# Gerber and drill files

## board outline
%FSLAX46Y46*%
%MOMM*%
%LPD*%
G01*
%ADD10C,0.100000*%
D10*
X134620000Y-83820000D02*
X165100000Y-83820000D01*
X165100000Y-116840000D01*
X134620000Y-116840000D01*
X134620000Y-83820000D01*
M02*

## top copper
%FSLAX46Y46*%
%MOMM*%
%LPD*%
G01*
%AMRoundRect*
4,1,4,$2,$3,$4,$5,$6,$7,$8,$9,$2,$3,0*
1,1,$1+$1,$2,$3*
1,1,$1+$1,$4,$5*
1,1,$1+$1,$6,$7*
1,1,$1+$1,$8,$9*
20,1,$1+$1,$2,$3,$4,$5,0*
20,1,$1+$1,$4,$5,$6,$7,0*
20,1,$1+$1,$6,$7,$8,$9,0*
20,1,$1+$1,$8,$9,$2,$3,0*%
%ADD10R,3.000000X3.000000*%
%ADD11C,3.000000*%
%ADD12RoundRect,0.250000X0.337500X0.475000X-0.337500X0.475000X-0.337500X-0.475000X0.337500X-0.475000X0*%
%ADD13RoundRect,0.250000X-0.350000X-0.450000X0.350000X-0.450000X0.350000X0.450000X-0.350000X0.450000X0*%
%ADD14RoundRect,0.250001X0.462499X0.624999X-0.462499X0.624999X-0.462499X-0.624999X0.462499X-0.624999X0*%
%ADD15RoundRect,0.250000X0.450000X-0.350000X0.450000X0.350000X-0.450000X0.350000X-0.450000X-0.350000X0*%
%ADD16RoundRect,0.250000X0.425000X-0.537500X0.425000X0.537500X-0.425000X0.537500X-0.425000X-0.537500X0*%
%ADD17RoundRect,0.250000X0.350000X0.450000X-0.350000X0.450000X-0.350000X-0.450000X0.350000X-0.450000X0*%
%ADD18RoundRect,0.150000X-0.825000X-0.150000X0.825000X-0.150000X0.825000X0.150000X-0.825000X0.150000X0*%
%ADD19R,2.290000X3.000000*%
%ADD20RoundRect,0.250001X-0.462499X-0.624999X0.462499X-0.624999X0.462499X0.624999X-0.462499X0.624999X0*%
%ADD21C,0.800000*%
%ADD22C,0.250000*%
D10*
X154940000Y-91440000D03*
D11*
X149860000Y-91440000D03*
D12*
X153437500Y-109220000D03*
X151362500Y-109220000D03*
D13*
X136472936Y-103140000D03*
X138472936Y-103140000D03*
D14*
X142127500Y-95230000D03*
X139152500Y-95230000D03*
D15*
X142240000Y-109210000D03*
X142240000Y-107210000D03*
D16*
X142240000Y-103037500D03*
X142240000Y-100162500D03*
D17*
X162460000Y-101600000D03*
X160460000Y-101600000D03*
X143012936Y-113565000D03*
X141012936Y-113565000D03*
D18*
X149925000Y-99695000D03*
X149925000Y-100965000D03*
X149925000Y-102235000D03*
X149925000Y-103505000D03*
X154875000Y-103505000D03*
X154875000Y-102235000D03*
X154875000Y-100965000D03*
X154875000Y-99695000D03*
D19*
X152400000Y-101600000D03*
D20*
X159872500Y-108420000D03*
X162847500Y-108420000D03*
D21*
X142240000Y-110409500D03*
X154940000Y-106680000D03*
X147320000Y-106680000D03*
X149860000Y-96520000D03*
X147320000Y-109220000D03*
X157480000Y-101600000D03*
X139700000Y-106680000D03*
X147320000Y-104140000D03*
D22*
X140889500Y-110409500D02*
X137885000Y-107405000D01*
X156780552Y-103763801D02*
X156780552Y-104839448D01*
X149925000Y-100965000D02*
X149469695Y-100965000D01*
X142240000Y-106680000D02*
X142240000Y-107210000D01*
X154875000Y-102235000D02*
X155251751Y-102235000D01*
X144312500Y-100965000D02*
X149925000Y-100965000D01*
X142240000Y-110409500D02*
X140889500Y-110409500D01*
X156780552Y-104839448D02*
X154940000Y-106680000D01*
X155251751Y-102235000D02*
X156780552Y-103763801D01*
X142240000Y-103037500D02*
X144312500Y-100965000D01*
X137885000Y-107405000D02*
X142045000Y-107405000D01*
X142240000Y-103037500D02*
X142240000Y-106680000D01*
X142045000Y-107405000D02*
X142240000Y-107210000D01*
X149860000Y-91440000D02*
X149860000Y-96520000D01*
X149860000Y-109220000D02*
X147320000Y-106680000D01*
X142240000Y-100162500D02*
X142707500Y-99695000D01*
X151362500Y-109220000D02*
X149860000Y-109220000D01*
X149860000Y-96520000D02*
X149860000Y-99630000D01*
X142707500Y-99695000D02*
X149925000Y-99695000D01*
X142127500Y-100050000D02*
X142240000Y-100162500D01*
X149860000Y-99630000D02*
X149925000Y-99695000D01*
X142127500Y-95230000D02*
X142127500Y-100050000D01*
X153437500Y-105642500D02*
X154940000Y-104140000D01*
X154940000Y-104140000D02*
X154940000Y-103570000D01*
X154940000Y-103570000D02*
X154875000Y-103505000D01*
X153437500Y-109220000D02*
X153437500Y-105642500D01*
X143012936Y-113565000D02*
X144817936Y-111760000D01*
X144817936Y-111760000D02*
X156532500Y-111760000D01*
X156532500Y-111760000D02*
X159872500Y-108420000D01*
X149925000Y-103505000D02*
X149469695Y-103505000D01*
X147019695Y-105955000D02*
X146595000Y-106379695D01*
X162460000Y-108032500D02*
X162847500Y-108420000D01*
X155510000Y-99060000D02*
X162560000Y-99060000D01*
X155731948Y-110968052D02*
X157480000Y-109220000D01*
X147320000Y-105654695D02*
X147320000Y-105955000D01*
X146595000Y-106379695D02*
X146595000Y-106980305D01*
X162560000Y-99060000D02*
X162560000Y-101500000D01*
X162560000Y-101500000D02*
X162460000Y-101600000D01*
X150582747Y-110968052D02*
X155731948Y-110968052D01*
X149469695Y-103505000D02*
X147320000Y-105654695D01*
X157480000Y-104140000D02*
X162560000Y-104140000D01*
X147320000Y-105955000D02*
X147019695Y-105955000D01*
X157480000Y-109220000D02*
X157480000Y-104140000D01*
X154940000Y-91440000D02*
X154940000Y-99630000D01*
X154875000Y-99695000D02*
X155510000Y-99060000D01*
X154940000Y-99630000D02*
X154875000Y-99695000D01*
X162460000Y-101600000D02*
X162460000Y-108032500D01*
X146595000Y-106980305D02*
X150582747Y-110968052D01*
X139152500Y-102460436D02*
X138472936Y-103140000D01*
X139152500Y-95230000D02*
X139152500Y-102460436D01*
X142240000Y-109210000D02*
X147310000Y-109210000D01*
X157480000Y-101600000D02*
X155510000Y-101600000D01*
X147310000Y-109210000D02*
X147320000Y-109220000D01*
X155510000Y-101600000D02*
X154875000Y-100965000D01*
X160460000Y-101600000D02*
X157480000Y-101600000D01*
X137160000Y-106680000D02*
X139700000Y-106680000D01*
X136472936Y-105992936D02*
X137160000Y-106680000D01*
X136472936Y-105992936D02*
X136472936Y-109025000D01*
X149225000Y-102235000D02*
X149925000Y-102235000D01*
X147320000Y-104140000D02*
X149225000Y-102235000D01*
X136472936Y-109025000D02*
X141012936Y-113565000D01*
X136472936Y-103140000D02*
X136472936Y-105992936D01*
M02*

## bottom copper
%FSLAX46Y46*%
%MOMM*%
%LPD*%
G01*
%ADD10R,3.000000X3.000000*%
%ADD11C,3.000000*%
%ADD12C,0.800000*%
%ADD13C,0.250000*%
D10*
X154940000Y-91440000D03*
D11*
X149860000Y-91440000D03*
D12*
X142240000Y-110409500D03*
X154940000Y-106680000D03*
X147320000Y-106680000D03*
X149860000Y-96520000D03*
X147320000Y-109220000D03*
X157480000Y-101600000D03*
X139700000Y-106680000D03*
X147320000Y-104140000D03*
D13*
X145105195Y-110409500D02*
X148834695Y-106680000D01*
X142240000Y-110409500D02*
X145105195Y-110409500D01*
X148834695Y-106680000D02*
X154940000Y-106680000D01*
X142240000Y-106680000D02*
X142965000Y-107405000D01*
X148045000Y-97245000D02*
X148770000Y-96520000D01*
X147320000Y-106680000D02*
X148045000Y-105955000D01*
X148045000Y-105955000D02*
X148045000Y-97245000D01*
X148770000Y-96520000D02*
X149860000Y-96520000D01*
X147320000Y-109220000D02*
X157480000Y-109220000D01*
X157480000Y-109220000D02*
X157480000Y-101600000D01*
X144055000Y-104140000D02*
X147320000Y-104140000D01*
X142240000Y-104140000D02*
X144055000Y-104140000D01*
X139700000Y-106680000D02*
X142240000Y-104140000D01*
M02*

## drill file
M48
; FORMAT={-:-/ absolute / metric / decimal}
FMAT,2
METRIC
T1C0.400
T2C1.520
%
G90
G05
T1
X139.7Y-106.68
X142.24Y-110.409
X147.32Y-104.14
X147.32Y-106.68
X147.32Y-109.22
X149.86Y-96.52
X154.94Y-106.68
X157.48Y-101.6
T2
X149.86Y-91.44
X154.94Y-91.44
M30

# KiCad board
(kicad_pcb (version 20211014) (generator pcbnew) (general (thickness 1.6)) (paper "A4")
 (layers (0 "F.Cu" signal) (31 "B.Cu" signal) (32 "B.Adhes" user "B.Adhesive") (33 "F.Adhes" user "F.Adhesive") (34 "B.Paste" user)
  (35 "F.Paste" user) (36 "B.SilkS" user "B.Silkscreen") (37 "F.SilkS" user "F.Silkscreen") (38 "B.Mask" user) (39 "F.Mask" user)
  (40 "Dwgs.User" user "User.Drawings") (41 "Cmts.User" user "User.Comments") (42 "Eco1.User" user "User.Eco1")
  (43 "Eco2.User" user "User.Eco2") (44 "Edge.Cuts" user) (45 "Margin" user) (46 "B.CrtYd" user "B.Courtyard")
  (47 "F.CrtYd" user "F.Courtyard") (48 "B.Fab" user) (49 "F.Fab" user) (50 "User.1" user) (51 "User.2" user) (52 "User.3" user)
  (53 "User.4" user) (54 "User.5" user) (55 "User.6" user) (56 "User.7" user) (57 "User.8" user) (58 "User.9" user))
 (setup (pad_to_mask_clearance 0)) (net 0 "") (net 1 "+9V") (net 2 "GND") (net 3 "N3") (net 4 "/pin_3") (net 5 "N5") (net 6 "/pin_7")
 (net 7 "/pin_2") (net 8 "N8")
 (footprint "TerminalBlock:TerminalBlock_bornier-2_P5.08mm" (layer "F.Cu") (at 154.94 91.44 180)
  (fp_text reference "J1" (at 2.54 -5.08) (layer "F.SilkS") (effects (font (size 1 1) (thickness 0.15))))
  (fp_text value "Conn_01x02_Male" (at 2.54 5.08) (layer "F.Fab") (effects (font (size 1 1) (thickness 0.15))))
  (pad "1" thru_hole rect (at 0 0 180) (size 3 3) (drill 1.52) (layers *.Cu *.Mask) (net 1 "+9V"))
  (pad "2" thru_hole circle (at 5.08 0 180) (size 3 3) (drill 1.52) (layers *.Cu *.Mask) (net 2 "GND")))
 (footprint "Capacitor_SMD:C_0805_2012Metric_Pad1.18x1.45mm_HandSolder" (layer "F.Cu") (at 152.4 109.22 180)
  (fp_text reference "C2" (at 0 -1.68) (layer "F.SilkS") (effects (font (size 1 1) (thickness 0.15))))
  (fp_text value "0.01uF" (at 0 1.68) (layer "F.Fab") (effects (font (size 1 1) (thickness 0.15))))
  (pad "1" smd roundrect (at -1.0375 0 180) (size 1.175 1.45) (layers "F.Cu" "F.Paste" "F.Mask") (roundrect_rratio 0.212766) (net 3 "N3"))
  (pad "2" smd roundrect (at 1.0375 0 180) (size 1.175 1.45) (layers "F.Cu" "F.Paste" "F.Mask") (roundrect_rratio 0.212766) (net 2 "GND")))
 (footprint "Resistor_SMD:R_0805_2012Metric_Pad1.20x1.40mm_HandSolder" (layer "F.Cu") (at 137.472936 103.14)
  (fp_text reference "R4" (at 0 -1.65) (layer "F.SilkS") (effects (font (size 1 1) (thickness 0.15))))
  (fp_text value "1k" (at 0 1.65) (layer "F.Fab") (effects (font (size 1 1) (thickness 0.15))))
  (pad "1" smd roundrect (at -1 0) (size 1.2 1.4) (layers "F.Cu" "F.Paste" "F.Mask") (roundrect_rratio 0.208333) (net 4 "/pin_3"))
  (pad "2" smd roundrect (at 1 0) (size 1.2 1.4) (layers "F.Cu" "F.Paste" "F.Mask") (roundrect_rratio 0.208333) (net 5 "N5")))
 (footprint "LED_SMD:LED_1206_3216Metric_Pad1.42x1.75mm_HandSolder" (layer "F.Cu") (at 140.64 95.23 180)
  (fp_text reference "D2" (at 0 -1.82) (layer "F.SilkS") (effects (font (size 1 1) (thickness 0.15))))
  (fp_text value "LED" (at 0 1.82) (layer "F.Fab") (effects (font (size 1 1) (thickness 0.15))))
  (pad "1" smd roundrect (at -1.4875 0 180) (size 1.425 1.75) (layers "F.Cu" "F.Paste" "F.Mask") (roundrect_rratio 0.175439) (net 2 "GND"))
  (pad "2" smd roundrect (at 1.4875 0 180) (size 1.425 1.75) (layers "F.Cu" "F.Paste" "F.Mask") (roundrect_rratio 0.175439) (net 5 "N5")))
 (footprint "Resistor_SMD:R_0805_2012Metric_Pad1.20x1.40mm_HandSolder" (layer "F.Cu") (at 142.24 108.21 90)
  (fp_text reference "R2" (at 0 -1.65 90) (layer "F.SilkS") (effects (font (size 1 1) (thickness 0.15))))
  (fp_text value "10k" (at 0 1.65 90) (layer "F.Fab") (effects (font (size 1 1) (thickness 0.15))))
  (pad "1" smd roundrect (at -1 0 90) (size 1.2 1.4) (layers "F.Cu" "F.Paste" "F.Mask") (roundrect_rratio 0.208333) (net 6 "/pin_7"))
  (pad "2" smd roundrect (at 1 0 90) (size 1.2 1.4) (layers "F.Cu" "F.Paste" "F.Mask") (roundrect_rratio 0.208333) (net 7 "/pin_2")))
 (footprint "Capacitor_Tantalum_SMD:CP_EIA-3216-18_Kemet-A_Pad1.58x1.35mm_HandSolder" (layer "F.Cu") (at 142.24 101.6 90)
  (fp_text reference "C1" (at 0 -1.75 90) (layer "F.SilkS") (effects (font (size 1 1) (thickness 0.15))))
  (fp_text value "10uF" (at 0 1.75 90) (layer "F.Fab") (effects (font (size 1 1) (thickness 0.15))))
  (pad "1" smd roundrect (at -1.4375 0 90) (size 1.575 1.35) (layers "F.Cu" "F.Paste" "F.Mask") (roundrect_rratio 0.185185) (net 7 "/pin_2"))
  (pad "2" smd roundrect (at 1.4375 0 90) (size 1.575 1.35) (layers "F.Cu" "F.Paste" "F.Mask") (roundrect_rratio 0.185185) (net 2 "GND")))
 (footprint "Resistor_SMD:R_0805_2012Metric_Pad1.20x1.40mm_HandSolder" (layer "F.Cu") (at 161.46 101.6 180)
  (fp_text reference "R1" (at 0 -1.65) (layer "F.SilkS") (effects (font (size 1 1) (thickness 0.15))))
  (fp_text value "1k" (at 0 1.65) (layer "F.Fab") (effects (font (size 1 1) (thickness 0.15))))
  (pad "1" smd roundrect (at -1 0 180) (size 1.2 1.4) (layers "F.Cu" "F.Paste" "F.Mask") (roundrect_rratio 0.208333) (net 1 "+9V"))
  (pad "2" smd roundrect (at 1 0 180) (size 1.2 1.4) (layers "F.Cu" "F.Paste" "F.Mask") (roundrect_rratio 0.208333) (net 6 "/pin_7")))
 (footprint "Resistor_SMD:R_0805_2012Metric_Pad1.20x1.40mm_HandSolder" (layer "F.Cu") (at 142.012936 113.565 180)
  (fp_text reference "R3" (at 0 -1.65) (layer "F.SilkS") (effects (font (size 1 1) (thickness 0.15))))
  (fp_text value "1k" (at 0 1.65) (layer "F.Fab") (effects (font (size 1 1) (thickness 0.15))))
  (pad "1" smd roundrect (at -1 0 180) (size 1.2 1.4) (layers "F.Cu" "F.Paste" "F.Mask") (roundrect_rratio 0.208333) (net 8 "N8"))
  (pad "2" smd roundrect (at 1 0 180) (size 1.2 1.4) (layers "F.Cu" "F.Paste" "F.Mask") (roundrect_rratio 0.208333) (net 4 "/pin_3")))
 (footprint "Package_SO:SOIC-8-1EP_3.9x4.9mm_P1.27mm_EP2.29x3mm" (layer "F.Cu") (at 152.4 101.6)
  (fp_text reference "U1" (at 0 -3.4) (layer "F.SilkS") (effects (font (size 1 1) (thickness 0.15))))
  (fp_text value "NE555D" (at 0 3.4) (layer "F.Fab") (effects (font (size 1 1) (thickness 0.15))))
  (pad "" smd roundrect (at -0.57 -0.75) (size 0.92 1.21) (layers "F.Paste") (roundrect_rratio 0.25))
  (pad "" smd roundrect (at -0.57 0.75) (size 0.92 1.21) (layers "F.Paste") (roundrect_rratio 0.25))
  (pad "" smd roundrect (at 0.57 -0.75) (size 0.92 1.21) (layers "F.Paste") (roundrect_rratio 0.25))
  (pad "" smd roundrect (at 0.57 0.75) (size 0.92 1.21) (layers "F.Paste") (roundrect_rratio 0.25))
  (pad "1" smd roundrect (at -2.475 -1.905) (size 1.95 0.6) (layers "F.Cu" "F.Paste" "F.Mask") (roundrect_rratio 0.25) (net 2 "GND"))
  (pad "2" smd roundrect (at -2.475 -0.635) (size 1.95 0.6) (layers "F.Cu" "F.Paste" "F.Mask") (roundrect_rratio 0.25) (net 7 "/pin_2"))
  (pad "3" smd roundrect (at -2.475 0.635) (size 1.95 0.6) (layers "F.Cu" "F.Paste" "F.Mask") (roundrect_rratio 0.25) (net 4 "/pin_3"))
  (pad "4" smd roundrect (at -2.475 1.905) (size 1.95 0.6) (layers "F.Cu" "F.Paste" "F.Mask") (roundrect_rratio 0.25) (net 1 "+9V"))
  (pad "5" smd roundrect (at 2.475 1.905) (size 1.95 0.6) (layers "F.Cu" "F.Paste" "F.Mask") (roundrect_rratio 0.25) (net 3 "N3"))
  (pad "6" smd roundrect (at 2.475 0.635) (size 1.95 0.6) (layers "F.Cu" "F.Paste" "F.Mask") (roundrect_rratio 0.25) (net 7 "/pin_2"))
  (pad "7" smd roundrect (at 2.475 -0.635) (size 1.95 0.6) (layers "F.Cu" "F.Paste" "F.Mask") (roundrect_rratio 0.25) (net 6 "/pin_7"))
  (pad "8" smd roundrect (at 2.475 -1.905) (size 1.95 0.6) (layers "F.Cu" "F.Paste" "F.Mask") (roundrect_rratio 0.25) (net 1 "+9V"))
  (pad "9" smd rect (at 0 0) (size 2.29 3) (layers "F.Cu" "F.Mask")))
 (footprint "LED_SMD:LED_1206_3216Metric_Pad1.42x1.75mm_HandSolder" (layer "F.Cu") (at 161.36 108.42)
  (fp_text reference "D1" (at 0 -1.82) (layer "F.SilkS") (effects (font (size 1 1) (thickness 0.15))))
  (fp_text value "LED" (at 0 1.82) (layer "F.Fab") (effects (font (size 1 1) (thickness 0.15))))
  (pad "1" smd roundrect (at -1.4875 0) (size 1.425 1.75) (layers "F.Cu" "F.Paste" "F.Mask") (roundrect_rratio 0.175439) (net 8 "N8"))
  (pad "2" smd roundrect (at 1.4875 0) (size 1.425 1.75) (layers "F.Cu" "F.Paste" "F.Mask") (roundrect_rratio 0.175439) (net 1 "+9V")))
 (gr_rect (start 134.62 83.82) (end 165.1 116.84) (layer "Edge.Cuts") (width 0.1) (fill none))
 (segment (start 140.8895 110.4095) (end 137.885 107.405) (width 0.25) (layer "F.Cu") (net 7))
 (segment (start 156.780552 103.763801) (end 156.780552 104.839448) (width 0.25) (layer "F.Cu") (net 7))
 (segment (start 149.925 100.965) (end 149.469695 100.965) (width 0.25) (layer "F.Cu") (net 7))
 (segment (start 142.24 106.68) (end 142.24 107.21) (width 0.25) (layer "F.Cu") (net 7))
 (segment (start 154.875 102.235) (end 155.251751 102.235) (width 0.25) (layer "F.Cu") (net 7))
 (segment (start 144.3125 100.965) (end 149.925 100.965) (width 0.25) (layer "F.Cu") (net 7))
 (segment (start 142.24 110.4095) (end 140.8895 110.4095) (width 0.25) (layer "F.Cu") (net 7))
 (segment (start 156.780552 104.839448) (end 154.94 106.68) (width 0.25) (layer "F.Cu") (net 7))
 (segment (start 155.251751 102.235) (end 156.780552 103.763801) (width 0.25) (layer "F.Cu") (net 7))
 (segment (start 142.24 103.0375) (end 144.3125 100.965) (width 0.25) (layer "F.Cu") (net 7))
 (segment (start 137.885 107.405) (end 142.045 107.405) (width 0.25) (layer "F.Cu") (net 7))
 (segment (start 142.24 103.0375) (end 142.24 106.68) (width 0.25) (layer "F.Cu") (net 7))
 (segment (start 142.045 107.405) (end 142.24 107.21) (width 0.25) (layer "F.Cu") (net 7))
 (via (at 142.24 110.4095) (size 0.8) (drill 0.4) (layers "F.Cu" "B.Cu") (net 7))
 (via (at 154.94 106.68) (size 0.8) (drill 0.4) (layers "F.Cu" "B.Cu") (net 7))
 (segment (start 145.105195 110.4095) (end 148.834695 106.68) (width 0.25) (layer "B.Cu") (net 7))
 (segment (start 142.24 110.4095) (end 145.105195 110.4095) (width 0.25) (layer "B.Cu") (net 7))
 (segment (start 148.834695 106.68) (end 154.94 106.68) (width 0.25) (layer "B.Cu") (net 7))
 (segment (start 142.24 106.68) (end 142.965 107.405) (width 0.25) (layer "B.Cu") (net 7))
 (segment (start 149.86 91.44) (end 149.86 96.52) (width 0.25) (layer "F.Cu") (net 2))
 (segment (start 149.86 109.22) (end 147.32 106.68) (width 0.25) (layer "F.Cu") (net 2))
 (segment (start 142.24 100.1625) (end 142.7075 99.695) (width 0.25) (layer "F.Cu") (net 2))
 (segment (start 151.3625 109.22) (end 149.86 109.22) (width 0.25) (layer "F.Cu") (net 2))
 (segment (start 149.86 96.52) (end 149.86 99.63) (width 0.25) (layer "F.Cu") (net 2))
 (segment (start 142.7075 99.695) (end 149.925 99.695) (width 0.25) (layer "F.Cu") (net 2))
 (segment (start 142.1275 100.05) (end 142.24 100.1625) (width 0.25) (layer "F.Cu") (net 2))
 (segment (start 149.86 99.63) (end 149.925 99.695) (width 0.25) (layer "F.Cu") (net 2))
 (segment (start 142.1275 95.23) (end 142.1275 100.05) (width 0.25) (layer "F.Cu") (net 2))
 (via (at 147.32 106.68) (size 0.8) (drill 0.4) (layers "F.Cu" "B.Cu") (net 2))
 (via (at 149.86 96.52) (size 0.8) (drill 0.4) (layers "F.Cu" "B.Cu") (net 2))
 (segment (start 148.045 97.245) (end 148.77 96.52) (width 0.25) (layer "B.Cu") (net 2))
 (segment (start 147.32 106.68) (end 148.045 105.955) (width 0.25) (layer "B.Cu") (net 2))
 (segment (start 148.045 105.955) (end 148.045 97.245) (width 0.25) (layer "B.Cu") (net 2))
 (segment (start 148.77 96.52) (end 149.86 96.52) (width 0.25) (layer "B.Cu") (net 2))
 (segment (start 153.4375 105.6425) (end 154.94 104.14) (width 0.25) (layer "F.Cu") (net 3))
 (segment (start 154.94 104.14) (end 154.94 103.57) (width 0.25) (layer "F.Cu") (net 3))
 (segment (start 154.94 103.57) (end 154.875 103.505) (width 0.25) (layer "F.Cu") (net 3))
 (segment (start 153.4375 109.22) (end 153.4375 105.6425) (width 0.25) (layer "F.Cu") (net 3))
 (segment (start 143.012936 113.565) (end 144.817936 111.76) (width 0.25) (layer "F.Cu") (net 8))
 (segment (start 144.817936 111.76) (end 156.5325 111.76) (width 0.25) (layer "F.Cu") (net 8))
 (segment (start 156.5325 111.76) (end 159.8725 108.42) (width 0.25) (layer "F.Cu") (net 8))
 (segment (start 149.925 103.505) (end 149.469695 103.505) (width 0.25) (layer "F.Cu") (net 1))
 (segment (start 147.019695 105.955) (end 146.595 106.379695) (width 0.25) (layer "F.Cu") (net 1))
 (segment (start 162.46 108.0325) (end 162.8475 108.42) (width 0.25) (layer "F.Cu") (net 1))
 (segment (start 155.51 99.06) (end 162.56 99.06) (width 0.25) (layer "F.Cu") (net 1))
 (segment (start 155.731948 110.968052) (end 157.48 109.22) (width 0.25) (layer "F.Cu") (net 1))
 (segment (start 147.32 105.654695) (end 147.32 105.955) (width 0.25) (layer "F.Cu") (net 1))
 (segment (start 146.595 106.379695) (end 146.595 106.980305) (width 0.25) (layer "F.Cu") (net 1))
 (segment (start 162.56 99.06) (end 162.56 101.5) (width 0.25) (layer "F.Cu") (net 1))
 (segment (start 162.56 101.5) (end 162.46 101.6) (width 0.25) (layer "F.Cu") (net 1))
 (segment (start 150.582747 110.968052) (end 155.731948 110.968052) (width 0.25) (layer "F.Cu") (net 1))
 (segment (start 149.469695 103.505) (end 147.32 105.654695) (width 0.25) (layer "F.Cu") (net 1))
 (segment (start 157.48 104.14) (end 162.56 104.14) (width 0.25) (layer "F.Cu") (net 1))
 (segment (start 147.32 105.955) (end 147.019695 105.955) (width 0.25) (layer "F.Cu") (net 1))
 (segment (start 157.48 109.22) (end 157.48 104.14) (width 0.25) (layer "F.Cu") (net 1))
 (segment (start 154.94 91.44) (end 154.94 99.63) (width 0.25) (layer "F.Cu") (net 1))
 (segment (start 154.875 99.695) (end 155.51 99.06) (width 0.25) (layer "F.Cu") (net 1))
 (segment (start 154.94 99.63) (end 154.875 99.695) (width 0.25) (layer "F.Cu") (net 1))
 (segment (start 162.46 101.6) (end 162.46 108.0325) (width 0.25) (layer "F.Cu") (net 1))
 (segment (start 146.595 106.980305) (end 150.582747 110.968052) (width 0.25) (layer "F.Cu") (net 1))
 (segment (start 139.1525 102.460436) (end 138.472936 103.14) (width 0.25) (layer "F.Cu") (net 5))
 (segment (start 139.1525 95.23) (end 139.1525 102.460436) (width 0.25) (layer "F.Cu") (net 5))
 (segment (start 142.24 109.21) (end 147.31 109.21) (width 0.25) (layer "F.Cu") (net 6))
 (segment (start 157.48 101.6) (end 155.51 101.6) (width 0.25) (layer "F.Cu") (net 6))
 (segment (start 147.31 109.21) (end 147.32 109.22) (width 0.25) (layer "F.Cu") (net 6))
 (segment (start 155.51 101.6) (end 154.875 100.965) (width 0.25) (layer "F.Cu") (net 6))
 (segment (start 160.46 101.6) (end 157.48 101.6) (width 0.25) (layer "F.Cu") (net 6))
 (via (at 147.32 109.22) (size 0.8) (drill 0.4) (layers "F.Cu" "B.Cu") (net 6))
 (via (at 157.48 101.6) (size 0.8) (drill 0.4) (layers "F.Cu" "B.Cu") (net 6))
 (segment (start 147.32 109.22) (end 157.48 109.22) (width 0.25) (layer "B.Cu") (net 6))
 (segment (start 157.48 109.22) (end 157.48 101.6) (width 0.25) (layer "B.Cu") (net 6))
 (segment (start 137.16 106.68) (end 139.7 106.68) (width 0.25) (layer "F.Cu") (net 4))
 (segment (start 136.472936 105.992936) (end 137.16 106.68) (width 0.25) (layer "F.Cu") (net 4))
 (segment (start 136.472936 105.992936) (end 136.472936 109.025) (width 0.25) (layer "F.Cu") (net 4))
 (segment (start 149.225 102.235) (end 149.925 102.235) (width 0.25) (layer "F.Cu") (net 4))
 (segment (start 147.32 104.14) (end 149.225 102.235) (width 0.25) (layer "F.Cu") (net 4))
 (segment (start 136.472936 109.025) (end 141.012936 113.565) (width 0.25) (layer "F.Cu") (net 4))
 (segment (start 136.472936 103.14) (end 136.472936 105.992936) (width 0.25) (layer "F.Cu") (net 4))
 (via (at 139.7 106.68) (size 0.8) (drill 0.4) (layers "F.Cu" "B.Cu") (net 4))
 (via (at 147.32 104.14) (size 0.8) (drill 0.4) (layers "F.Cu" "B.Cu") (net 4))
 (segment (start 144.055 104.14) (end 147.32 104.14) (width 0.25) (layer "B.Cu") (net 4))
 (segment (start 142.24 104.14) (end 144.055 104.14) (width 0.25) (layer "B.Cu") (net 4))
 (segment (start 139.7 106.68) (end 142.24 104.14) (width 0.25) (layer "B.Cu") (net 4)))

